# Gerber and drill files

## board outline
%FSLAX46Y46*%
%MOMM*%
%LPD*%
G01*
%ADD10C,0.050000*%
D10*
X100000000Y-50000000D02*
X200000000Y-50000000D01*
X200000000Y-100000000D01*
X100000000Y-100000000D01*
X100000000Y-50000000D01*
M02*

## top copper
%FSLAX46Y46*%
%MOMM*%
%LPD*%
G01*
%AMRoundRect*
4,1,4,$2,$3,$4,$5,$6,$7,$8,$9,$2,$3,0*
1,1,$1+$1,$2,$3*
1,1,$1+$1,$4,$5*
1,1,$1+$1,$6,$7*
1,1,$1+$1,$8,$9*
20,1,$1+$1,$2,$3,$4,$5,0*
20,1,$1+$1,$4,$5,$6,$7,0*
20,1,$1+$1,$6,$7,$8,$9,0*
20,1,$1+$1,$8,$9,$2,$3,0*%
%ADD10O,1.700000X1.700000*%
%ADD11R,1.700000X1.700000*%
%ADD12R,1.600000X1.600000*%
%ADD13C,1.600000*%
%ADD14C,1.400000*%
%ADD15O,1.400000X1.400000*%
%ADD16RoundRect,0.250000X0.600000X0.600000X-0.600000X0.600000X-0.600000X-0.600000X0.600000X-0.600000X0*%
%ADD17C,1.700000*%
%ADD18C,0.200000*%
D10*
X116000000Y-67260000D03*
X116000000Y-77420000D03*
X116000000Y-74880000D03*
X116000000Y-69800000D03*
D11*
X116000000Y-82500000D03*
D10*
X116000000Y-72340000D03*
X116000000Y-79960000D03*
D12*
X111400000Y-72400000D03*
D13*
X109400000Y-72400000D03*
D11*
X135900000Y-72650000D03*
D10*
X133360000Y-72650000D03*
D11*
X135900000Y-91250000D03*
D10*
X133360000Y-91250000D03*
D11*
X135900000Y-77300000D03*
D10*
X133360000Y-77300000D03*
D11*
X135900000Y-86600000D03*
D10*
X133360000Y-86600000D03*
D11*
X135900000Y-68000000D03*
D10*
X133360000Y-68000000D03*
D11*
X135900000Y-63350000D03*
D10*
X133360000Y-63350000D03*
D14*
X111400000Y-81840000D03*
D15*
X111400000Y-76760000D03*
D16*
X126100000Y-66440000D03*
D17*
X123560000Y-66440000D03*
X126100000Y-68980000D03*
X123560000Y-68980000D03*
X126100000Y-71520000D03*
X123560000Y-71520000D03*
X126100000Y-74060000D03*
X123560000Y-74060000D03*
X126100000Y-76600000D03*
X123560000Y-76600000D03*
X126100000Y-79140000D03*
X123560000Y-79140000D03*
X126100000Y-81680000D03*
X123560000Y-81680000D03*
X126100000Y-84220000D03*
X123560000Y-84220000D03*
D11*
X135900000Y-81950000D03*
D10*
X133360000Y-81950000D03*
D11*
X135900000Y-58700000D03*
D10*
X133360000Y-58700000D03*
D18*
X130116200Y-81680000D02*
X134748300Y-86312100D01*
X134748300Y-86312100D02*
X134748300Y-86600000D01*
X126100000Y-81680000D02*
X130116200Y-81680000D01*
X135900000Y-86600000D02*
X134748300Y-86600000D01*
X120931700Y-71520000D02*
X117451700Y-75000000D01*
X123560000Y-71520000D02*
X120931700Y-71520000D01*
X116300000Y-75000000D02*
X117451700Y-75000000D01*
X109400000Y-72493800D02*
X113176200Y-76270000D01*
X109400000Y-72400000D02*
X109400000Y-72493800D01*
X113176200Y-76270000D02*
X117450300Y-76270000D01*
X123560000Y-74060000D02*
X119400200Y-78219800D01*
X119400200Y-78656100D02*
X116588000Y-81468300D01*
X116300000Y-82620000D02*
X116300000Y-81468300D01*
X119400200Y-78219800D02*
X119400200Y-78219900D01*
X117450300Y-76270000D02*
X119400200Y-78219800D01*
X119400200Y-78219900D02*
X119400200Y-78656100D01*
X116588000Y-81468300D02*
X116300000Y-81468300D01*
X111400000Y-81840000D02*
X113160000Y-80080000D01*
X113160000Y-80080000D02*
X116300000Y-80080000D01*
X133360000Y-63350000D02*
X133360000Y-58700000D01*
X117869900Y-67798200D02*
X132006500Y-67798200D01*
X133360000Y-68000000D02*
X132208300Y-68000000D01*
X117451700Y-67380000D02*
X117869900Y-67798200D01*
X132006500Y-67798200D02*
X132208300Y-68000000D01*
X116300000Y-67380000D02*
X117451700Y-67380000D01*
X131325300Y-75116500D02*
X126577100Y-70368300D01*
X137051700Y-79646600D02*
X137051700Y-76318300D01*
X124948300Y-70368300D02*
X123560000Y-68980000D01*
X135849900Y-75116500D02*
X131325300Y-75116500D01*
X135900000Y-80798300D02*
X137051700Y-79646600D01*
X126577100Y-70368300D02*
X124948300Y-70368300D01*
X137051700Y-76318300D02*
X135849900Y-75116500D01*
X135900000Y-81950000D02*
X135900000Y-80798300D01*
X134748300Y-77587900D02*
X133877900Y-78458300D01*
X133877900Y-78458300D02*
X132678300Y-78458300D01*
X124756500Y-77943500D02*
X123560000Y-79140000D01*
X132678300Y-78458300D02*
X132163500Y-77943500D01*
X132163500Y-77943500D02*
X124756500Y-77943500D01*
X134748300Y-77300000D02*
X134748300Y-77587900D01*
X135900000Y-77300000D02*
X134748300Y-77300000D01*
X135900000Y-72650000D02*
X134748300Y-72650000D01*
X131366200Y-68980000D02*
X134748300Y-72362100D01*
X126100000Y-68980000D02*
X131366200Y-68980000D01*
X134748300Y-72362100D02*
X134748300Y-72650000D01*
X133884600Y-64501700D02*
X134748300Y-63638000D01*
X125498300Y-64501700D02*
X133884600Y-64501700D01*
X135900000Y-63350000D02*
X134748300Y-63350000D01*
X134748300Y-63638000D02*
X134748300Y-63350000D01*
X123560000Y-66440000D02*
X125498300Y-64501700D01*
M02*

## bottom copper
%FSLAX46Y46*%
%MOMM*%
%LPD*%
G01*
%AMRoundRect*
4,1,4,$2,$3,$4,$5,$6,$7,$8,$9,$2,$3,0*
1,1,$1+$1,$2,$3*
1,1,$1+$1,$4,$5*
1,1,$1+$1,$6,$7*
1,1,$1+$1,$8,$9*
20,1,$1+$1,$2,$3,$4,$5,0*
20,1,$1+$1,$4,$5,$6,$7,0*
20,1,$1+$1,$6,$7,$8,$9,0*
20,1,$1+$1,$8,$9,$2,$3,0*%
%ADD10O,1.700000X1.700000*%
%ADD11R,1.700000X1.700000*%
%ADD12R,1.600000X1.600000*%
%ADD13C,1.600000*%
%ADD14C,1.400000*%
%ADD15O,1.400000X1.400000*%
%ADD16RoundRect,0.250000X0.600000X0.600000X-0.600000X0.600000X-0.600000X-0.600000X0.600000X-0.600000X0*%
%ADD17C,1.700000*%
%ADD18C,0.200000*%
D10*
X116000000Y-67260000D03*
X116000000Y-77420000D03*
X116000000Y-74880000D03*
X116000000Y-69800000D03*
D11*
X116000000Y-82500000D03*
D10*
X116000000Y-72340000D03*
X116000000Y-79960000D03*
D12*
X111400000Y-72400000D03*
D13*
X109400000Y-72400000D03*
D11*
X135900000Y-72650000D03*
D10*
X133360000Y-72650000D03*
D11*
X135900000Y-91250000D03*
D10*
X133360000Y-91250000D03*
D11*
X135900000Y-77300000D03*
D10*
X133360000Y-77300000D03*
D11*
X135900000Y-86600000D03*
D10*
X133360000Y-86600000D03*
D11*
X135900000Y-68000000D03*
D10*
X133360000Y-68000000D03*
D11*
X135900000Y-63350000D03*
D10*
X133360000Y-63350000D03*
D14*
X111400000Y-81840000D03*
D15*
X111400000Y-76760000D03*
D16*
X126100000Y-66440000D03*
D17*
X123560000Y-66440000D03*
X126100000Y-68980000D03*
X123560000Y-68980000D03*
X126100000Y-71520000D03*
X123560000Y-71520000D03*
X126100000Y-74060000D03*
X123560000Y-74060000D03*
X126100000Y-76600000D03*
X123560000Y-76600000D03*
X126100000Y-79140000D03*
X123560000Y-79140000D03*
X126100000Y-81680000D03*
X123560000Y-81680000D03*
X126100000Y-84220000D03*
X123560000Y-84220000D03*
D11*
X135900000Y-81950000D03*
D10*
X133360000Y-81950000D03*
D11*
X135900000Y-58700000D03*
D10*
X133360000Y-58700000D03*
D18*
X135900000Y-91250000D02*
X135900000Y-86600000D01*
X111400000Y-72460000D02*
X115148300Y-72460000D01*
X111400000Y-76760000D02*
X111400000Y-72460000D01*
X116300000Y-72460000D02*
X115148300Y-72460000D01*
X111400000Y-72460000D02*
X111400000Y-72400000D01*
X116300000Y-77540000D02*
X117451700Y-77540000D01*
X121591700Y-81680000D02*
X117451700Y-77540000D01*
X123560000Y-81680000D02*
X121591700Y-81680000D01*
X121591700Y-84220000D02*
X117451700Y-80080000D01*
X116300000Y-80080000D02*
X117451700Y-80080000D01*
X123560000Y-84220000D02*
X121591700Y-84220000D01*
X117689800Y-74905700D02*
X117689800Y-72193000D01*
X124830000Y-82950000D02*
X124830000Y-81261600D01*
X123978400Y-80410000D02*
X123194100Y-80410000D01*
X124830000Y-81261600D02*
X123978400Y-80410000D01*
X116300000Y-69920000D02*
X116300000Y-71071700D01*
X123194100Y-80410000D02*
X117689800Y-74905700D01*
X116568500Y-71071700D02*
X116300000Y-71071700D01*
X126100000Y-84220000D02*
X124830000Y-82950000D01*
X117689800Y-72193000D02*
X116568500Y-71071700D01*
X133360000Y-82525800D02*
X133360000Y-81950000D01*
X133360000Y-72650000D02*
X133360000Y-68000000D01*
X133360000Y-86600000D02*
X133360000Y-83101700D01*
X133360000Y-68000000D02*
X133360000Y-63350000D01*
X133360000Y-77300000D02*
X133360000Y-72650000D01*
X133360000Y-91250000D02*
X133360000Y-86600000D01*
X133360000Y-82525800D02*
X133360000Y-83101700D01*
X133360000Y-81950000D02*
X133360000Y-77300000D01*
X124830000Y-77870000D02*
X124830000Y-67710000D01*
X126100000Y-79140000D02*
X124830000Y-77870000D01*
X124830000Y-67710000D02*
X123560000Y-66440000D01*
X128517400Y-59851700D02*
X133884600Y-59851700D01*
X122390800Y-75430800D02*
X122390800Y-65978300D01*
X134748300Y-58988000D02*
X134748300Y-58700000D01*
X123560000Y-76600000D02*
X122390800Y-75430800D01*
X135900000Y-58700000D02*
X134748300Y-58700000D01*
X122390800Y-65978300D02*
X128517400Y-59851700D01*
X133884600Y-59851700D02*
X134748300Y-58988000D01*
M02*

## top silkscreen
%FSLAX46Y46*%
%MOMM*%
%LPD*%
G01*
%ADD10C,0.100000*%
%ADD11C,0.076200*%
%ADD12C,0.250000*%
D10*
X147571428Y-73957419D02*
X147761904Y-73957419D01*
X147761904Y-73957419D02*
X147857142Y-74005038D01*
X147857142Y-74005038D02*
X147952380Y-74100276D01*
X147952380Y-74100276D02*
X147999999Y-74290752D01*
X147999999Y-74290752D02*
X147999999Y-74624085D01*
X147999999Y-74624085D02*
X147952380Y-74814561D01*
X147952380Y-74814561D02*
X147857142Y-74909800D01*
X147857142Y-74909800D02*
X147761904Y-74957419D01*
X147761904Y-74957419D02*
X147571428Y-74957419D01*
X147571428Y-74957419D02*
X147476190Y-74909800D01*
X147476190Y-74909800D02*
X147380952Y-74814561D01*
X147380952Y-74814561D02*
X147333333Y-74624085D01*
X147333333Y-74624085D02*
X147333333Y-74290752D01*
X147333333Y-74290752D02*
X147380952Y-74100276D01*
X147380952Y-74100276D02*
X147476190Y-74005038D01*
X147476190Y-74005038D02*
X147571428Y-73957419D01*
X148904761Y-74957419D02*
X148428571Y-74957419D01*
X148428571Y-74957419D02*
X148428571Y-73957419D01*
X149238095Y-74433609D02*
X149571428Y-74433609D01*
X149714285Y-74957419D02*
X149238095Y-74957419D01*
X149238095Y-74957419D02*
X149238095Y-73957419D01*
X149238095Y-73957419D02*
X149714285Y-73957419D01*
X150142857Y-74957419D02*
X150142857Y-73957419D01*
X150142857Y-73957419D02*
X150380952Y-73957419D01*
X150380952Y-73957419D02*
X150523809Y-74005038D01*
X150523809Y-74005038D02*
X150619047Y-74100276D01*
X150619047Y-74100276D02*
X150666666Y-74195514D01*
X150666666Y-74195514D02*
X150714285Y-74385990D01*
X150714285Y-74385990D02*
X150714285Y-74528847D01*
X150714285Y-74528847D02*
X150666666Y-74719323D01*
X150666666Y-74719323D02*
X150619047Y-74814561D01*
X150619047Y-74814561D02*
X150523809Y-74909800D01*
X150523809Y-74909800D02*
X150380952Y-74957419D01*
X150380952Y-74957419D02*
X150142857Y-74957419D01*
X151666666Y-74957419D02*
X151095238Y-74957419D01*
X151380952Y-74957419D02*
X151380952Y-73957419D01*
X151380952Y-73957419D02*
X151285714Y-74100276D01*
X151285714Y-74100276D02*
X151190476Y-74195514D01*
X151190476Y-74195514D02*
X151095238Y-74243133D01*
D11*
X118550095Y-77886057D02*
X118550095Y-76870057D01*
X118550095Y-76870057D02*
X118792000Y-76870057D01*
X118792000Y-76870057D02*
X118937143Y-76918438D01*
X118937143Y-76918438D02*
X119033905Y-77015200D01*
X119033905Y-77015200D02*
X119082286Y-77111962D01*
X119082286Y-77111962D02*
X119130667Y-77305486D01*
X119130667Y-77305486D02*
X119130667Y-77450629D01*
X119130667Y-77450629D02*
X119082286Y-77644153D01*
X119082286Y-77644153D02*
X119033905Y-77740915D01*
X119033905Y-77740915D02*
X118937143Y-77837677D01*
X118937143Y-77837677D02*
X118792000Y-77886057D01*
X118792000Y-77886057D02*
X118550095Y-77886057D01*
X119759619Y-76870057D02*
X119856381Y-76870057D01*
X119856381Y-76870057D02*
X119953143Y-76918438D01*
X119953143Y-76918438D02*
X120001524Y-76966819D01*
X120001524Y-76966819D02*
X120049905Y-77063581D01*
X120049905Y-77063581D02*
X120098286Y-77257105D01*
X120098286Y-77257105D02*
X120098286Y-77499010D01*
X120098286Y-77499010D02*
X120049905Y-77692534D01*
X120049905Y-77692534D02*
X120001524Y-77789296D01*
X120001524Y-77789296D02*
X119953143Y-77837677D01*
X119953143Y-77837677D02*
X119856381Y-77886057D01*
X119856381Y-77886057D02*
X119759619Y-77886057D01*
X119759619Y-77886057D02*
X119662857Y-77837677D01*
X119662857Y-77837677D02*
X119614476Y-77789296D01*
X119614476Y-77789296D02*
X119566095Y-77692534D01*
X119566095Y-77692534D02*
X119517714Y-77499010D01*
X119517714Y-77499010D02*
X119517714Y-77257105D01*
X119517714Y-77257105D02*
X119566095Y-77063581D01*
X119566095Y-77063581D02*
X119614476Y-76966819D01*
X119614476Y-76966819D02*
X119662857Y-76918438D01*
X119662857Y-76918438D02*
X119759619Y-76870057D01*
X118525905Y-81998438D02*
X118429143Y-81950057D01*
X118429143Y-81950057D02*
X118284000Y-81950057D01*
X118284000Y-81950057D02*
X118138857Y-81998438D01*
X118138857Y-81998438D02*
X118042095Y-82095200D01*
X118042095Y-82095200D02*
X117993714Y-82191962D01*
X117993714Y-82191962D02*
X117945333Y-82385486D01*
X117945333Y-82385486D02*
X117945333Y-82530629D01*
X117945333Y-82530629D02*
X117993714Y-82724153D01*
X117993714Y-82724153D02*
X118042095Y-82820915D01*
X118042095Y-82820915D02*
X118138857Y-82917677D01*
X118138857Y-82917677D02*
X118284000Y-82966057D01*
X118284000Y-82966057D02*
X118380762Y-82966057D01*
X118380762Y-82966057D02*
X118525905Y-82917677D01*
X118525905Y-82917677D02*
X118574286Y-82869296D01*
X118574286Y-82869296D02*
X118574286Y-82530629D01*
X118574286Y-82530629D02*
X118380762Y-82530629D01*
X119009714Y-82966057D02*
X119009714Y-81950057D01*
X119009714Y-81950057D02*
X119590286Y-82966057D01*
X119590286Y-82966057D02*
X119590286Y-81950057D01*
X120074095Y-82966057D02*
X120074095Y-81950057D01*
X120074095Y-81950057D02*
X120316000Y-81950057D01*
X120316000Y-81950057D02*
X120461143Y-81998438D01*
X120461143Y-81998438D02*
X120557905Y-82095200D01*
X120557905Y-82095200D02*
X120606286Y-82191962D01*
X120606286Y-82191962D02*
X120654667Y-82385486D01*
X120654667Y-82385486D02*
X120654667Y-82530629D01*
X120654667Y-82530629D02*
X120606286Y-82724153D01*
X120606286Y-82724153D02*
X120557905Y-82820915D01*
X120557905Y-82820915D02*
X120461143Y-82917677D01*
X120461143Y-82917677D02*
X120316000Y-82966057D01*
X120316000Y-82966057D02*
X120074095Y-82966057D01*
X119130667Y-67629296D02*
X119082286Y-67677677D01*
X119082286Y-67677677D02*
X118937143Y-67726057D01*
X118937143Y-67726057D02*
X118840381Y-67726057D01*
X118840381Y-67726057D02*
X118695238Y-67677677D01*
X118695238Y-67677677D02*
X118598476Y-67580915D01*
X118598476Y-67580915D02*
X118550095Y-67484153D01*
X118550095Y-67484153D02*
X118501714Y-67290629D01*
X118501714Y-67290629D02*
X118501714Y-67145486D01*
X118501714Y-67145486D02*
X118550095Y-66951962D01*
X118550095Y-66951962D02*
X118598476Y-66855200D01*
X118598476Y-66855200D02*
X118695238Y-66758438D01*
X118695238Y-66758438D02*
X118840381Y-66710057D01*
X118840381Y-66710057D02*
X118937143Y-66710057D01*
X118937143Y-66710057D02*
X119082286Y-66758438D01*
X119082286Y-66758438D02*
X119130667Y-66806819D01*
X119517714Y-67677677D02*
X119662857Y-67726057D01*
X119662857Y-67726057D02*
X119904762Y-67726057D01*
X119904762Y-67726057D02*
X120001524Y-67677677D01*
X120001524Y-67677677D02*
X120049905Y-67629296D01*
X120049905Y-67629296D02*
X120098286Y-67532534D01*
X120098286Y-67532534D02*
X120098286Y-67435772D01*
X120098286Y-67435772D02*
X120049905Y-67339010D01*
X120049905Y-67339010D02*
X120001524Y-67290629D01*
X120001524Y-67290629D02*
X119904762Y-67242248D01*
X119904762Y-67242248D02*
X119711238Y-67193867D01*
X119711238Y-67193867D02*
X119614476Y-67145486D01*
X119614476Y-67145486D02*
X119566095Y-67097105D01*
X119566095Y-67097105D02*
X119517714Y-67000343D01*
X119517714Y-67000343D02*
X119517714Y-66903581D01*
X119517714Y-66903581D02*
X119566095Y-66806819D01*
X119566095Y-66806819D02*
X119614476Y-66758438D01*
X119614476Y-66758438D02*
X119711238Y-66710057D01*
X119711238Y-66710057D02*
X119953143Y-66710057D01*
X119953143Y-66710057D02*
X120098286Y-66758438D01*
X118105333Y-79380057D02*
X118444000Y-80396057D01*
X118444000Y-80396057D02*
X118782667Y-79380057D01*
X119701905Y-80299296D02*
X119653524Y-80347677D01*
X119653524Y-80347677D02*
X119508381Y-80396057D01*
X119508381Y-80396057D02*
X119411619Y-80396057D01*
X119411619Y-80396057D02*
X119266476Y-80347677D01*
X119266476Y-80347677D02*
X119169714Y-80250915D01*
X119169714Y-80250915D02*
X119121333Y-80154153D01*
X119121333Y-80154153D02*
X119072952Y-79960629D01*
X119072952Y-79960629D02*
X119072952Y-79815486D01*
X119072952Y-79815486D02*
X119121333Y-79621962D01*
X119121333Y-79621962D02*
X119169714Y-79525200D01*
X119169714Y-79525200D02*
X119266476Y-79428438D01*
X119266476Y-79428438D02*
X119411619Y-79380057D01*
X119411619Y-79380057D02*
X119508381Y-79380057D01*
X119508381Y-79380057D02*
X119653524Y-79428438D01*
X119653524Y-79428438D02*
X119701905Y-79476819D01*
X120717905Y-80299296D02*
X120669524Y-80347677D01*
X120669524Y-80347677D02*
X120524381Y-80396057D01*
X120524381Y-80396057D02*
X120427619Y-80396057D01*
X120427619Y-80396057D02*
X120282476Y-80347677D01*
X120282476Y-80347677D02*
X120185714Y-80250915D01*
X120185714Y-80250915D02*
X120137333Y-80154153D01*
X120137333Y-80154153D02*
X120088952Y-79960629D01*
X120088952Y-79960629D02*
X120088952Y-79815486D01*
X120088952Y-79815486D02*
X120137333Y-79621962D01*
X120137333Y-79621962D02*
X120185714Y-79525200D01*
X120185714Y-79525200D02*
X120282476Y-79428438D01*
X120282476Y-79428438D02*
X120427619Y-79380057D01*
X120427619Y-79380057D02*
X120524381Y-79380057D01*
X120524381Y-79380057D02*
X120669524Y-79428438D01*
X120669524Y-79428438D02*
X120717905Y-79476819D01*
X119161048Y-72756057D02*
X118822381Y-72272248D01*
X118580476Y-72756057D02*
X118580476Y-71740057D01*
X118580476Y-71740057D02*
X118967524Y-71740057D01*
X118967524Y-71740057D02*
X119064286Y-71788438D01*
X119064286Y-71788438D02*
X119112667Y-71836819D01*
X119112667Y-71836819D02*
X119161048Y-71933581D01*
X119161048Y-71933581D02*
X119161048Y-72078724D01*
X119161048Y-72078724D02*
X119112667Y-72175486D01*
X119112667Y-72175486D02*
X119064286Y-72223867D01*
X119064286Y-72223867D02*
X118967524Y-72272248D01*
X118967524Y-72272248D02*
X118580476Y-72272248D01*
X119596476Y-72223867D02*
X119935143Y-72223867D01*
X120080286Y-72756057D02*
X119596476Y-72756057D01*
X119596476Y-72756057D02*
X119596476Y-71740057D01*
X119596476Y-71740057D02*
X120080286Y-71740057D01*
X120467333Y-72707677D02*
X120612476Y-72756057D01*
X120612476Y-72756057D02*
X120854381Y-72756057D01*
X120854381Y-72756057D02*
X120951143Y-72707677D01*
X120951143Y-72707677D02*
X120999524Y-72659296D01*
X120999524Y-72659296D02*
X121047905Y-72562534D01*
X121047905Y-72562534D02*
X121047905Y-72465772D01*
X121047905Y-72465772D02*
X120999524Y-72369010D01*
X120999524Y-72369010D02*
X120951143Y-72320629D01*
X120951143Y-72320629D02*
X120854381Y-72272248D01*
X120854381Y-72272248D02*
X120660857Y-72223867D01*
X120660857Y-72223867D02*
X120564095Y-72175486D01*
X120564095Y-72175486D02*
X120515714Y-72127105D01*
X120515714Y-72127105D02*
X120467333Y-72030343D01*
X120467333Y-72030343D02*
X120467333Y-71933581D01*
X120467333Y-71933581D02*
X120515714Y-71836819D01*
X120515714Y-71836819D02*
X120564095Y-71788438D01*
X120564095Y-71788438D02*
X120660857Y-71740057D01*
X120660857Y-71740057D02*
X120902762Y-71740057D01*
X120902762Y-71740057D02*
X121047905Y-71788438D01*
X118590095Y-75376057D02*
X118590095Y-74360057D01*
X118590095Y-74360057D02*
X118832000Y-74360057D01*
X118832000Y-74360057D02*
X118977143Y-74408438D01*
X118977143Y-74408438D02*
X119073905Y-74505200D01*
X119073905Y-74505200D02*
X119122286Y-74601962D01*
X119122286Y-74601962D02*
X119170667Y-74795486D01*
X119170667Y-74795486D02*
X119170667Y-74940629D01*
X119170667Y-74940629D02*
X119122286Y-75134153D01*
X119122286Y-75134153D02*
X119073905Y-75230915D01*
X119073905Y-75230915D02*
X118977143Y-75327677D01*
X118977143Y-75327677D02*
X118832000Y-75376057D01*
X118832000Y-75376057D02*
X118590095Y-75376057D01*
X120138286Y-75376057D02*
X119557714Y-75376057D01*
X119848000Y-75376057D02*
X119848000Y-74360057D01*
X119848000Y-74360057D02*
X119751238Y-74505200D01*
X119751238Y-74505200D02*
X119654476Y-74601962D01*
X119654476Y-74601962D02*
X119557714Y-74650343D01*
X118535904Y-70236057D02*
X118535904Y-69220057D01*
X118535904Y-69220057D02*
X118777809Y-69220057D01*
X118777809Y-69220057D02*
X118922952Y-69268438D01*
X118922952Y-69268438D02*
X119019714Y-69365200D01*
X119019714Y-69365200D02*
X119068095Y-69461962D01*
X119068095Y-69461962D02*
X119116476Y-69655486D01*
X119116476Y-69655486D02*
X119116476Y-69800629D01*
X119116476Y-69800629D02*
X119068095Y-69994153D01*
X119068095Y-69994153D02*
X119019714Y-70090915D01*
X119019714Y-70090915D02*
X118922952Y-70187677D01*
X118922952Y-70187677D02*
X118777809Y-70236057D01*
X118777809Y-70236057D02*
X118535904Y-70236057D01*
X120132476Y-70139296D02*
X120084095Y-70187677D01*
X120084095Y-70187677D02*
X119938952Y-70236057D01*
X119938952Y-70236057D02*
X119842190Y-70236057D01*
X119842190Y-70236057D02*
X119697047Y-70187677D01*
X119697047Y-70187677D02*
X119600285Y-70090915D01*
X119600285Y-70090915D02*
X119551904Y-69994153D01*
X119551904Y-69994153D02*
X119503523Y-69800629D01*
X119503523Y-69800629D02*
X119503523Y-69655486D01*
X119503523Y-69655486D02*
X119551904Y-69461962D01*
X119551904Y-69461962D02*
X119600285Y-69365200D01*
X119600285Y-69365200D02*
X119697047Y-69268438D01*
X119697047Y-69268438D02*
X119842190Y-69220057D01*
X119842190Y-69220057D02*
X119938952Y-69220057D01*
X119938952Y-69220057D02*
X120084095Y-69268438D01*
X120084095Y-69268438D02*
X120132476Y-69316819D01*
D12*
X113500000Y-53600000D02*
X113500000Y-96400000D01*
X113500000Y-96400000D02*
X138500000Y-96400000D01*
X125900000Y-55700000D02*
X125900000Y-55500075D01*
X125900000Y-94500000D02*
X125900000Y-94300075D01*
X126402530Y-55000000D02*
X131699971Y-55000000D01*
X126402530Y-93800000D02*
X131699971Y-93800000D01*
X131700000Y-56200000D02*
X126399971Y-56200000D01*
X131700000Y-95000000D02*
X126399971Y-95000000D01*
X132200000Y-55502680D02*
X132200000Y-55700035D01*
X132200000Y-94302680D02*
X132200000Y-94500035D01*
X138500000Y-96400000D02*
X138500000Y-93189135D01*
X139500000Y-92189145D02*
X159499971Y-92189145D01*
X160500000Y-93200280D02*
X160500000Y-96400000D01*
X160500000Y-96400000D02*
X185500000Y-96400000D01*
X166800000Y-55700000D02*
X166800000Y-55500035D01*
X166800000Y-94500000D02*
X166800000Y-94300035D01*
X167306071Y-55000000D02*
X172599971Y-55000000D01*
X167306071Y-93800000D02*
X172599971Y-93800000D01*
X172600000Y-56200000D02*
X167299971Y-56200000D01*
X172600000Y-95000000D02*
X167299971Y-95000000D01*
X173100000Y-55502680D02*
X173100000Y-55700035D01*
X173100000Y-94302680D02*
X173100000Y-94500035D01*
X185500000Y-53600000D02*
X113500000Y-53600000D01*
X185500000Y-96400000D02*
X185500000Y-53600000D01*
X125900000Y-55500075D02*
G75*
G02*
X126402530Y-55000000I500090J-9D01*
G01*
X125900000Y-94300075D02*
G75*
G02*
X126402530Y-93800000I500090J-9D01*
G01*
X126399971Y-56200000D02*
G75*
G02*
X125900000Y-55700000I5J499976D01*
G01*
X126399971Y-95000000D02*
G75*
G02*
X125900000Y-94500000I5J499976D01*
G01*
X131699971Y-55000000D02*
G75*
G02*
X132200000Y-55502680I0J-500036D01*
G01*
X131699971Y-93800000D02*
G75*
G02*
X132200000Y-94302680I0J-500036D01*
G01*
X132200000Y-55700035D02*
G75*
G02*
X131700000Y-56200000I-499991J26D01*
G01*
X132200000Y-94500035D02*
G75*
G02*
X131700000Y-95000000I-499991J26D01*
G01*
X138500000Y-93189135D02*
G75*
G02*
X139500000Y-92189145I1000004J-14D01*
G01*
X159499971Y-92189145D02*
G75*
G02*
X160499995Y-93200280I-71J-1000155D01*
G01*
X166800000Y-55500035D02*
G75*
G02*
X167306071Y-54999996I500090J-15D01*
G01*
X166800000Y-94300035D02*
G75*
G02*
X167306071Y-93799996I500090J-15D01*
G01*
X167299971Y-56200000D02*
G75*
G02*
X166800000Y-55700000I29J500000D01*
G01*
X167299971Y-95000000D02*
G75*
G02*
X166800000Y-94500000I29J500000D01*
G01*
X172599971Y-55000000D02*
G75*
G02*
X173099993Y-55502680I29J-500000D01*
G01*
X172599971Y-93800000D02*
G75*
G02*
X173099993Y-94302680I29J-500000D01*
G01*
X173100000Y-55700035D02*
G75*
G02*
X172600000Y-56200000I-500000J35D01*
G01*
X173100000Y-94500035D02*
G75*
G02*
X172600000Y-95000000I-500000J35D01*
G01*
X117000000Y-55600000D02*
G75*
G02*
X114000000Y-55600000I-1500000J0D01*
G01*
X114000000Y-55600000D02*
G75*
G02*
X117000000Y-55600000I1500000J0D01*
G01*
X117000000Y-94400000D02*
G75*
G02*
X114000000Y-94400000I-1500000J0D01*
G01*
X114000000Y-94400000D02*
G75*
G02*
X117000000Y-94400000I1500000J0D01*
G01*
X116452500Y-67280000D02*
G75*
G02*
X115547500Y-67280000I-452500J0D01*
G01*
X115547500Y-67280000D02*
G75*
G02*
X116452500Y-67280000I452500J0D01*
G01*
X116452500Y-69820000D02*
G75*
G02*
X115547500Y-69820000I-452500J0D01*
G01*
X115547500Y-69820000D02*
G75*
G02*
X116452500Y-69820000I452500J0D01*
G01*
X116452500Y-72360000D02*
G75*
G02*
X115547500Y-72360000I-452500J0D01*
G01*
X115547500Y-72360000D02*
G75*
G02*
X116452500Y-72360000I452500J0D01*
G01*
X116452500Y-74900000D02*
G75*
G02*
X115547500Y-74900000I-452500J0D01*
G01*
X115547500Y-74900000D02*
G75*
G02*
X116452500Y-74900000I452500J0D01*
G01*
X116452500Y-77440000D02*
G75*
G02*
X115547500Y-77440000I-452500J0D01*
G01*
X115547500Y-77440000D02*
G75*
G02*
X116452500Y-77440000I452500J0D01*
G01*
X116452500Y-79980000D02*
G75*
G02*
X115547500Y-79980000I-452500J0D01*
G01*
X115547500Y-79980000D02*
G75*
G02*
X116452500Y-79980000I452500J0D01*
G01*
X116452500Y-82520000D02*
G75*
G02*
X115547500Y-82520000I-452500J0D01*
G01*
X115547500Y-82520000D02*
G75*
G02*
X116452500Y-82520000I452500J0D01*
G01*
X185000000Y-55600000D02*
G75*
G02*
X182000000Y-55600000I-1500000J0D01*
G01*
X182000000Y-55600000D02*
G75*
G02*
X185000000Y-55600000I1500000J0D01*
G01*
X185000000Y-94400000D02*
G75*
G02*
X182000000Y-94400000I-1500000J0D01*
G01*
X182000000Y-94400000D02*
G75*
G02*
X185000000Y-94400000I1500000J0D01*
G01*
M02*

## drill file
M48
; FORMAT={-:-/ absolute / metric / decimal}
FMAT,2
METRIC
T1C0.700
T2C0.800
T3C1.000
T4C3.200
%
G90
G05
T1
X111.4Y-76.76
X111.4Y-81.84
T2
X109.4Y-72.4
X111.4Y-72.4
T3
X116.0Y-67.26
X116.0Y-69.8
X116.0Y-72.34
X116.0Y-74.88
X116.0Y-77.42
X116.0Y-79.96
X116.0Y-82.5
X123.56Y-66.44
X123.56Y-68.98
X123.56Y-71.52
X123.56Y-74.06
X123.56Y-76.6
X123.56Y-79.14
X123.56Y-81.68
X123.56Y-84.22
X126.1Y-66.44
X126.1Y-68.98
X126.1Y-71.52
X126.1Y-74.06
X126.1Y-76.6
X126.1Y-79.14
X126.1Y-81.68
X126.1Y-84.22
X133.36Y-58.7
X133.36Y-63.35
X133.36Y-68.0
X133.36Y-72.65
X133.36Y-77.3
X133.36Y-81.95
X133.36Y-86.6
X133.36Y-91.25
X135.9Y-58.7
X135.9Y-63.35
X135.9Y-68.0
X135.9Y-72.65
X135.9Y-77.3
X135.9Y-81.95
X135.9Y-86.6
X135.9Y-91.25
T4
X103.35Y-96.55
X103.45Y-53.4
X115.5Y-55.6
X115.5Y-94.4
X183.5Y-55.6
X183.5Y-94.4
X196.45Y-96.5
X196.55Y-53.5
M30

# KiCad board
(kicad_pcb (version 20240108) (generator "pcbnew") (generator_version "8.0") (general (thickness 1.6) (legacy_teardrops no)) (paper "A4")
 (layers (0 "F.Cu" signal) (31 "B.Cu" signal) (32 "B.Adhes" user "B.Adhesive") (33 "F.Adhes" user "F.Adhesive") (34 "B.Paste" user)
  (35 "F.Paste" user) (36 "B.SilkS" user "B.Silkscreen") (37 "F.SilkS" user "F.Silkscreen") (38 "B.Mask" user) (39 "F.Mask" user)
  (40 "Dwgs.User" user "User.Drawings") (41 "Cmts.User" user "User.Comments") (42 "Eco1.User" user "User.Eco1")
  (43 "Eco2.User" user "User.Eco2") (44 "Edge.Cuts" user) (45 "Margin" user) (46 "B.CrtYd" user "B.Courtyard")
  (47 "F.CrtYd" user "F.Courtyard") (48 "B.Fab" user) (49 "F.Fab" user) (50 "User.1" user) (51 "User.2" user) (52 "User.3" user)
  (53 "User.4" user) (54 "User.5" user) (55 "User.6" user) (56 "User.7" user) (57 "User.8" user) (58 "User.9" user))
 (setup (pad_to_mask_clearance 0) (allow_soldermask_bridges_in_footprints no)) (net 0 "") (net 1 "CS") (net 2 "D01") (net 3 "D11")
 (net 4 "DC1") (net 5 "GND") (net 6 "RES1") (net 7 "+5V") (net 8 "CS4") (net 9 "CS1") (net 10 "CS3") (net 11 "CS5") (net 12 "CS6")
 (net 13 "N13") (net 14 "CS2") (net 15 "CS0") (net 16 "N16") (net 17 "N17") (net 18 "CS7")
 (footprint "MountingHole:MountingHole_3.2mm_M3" (layer "F.Cu") (at 183.5 55.6)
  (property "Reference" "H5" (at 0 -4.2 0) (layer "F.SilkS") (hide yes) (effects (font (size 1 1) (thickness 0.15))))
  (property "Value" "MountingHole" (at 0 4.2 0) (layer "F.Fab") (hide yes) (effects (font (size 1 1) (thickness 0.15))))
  (pad "" np_thru_hole circle (at 0 0) (size 3.2 3.2) (drill 3.2) (layers "*.Cu" "*.Mask")))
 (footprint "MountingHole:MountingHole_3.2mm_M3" (layer "F.Cu") (at 183.5 94.4)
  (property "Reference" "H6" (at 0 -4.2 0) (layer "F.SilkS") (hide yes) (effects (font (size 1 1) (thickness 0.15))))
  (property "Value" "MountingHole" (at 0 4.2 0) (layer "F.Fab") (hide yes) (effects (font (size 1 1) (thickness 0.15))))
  (pad "" np_thru_hole circle (at 0 0) (size 3.2 3.2) (drill 3.2) (layers "*.Cu" "*.Mask")))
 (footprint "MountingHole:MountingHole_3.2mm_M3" (layer "F.Cu") (at 196.55 53.5)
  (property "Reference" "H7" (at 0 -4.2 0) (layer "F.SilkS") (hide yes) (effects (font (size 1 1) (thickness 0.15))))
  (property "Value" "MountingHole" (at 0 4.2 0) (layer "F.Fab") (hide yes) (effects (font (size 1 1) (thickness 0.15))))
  (pad "" np_thru_hole circle (at 0 0) (size 3.2 3.2) (drill 3.2) (layers "*.Cu" "*.Mask")))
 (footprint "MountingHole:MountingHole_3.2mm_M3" (layer "F.Cu") (at 115.5 55.6)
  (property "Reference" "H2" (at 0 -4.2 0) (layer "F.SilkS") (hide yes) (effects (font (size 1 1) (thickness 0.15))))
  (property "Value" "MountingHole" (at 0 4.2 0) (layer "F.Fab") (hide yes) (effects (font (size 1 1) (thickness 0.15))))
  (pad "" np_thru_hole circle (at 0 0) (size 3.2 3.2) (drill 3.2) (layers "*.Cu" "*.Mask")))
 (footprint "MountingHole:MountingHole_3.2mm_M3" (layer "F.Cu") (at 103.35 96.55)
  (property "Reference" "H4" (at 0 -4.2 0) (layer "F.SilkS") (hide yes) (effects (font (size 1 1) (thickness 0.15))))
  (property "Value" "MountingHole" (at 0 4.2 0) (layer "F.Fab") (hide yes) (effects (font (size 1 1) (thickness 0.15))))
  (pad "" np_thru_hole circle (at 0 0) (size 3.2 3.2) (drill 3.2) (layers "*.Cu" "*.Mask")))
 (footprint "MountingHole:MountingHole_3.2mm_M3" (layer "F.Cu") (at 103.45 53.4)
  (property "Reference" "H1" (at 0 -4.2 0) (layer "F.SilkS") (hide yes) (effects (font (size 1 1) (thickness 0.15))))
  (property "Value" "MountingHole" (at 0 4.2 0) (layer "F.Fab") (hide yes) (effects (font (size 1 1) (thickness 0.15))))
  (pad "" np_thru_hole circle (at 0 0) (size 3.2 3.2) (drill 3.2) (layers "*.Cu" "*.Mask")))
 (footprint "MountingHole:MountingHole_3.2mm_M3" (layer "F.Cu") (at 115.5 94.4)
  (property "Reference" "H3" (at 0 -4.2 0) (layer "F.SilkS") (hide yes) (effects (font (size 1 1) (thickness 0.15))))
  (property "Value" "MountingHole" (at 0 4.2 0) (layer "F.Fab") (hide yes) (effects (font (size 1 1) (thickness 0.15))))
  (pad "" np_thru_hole circle (at 0 0) (size 3.2 3.2) (drill 3.2) (layers "*.Cu" "*.Mask")))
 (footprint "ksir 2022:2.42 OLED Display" (layer "F.Cu") (at 149.5 75)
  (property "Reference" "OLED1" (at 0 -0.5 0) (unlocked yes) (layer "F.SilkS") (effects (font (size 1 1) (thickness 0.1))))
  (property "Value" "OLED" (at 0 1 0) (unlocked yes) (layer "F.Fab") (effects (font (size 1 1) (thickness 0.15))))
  (fp_line (start -36 -21.4) (end -36 21.4) (stroke (width 0.25) (type default)) (layer "F.SilkS"))
  (fp_line (start -36 21.4) (end -11 21.4) (stroke (width 0.25) (type default)) (layer "F.SilkS"))
  (fp_line (start -23.6 -19.3) (end -23.6 -19.499925) (stroke (width 0.25) (type default)) (layer "F.SilkS"))
  (fp_line (start -23.6 19.5) (end -23.6 19.300075) (stroke (width 0.25) (type default)) (layer "F.SilkS"))
  (fp_line (start -23.09747 -20) (end -17.800029 -20) (stroke (width 0.25) (type default)) (layer "F.SilkS"))
  (fp_line (start -23.09747 18.8) (end -17.800029 18.8) (stroke (width 0.25) (type default)) (layer "F.SilkS"))
  (fp_line (start -17.8 -18.8) (end -23.100029 -18.8) (stroke (width 0.25) (type default)) (layer "F.SilkS"))
  (fp_line (start -17.8 20) (end -23.100029 20) (stroke (width 0.25) (type default)) (layer "F.SilkS"))
  (fp_line (start -17.3 -19.49732) (end -17.3 -19.299965) (stroke (width 0.25) (type default)) (layer "F.SilkS"))
  (fp_line (start -17.3 19.30268) (end -17.3 19.500035) (stroke (width 0.25) (type default)) (layer "F.SilkS"))
  (fp_line (start -11 21.4) (end -11 18.189135) (stroke (width 0.25) (type default)) (layer "F.SilkS"))
  (fp_line (start -10 17.189145) (end 9.999971 17.189145) (stroke (width 0.25) (type default)) (layer "F.SilkS"))
  (fp_line (start 11 18.20028) (end 11 21.4) (stroke (width 0.25) (type default)) (layer "F.SilkS"))
  (fp_line (start 11 21.4) (end 36 21.4) (stroke (width 0.25) (type default)) (layer "F.SilkS"))
  (fp_line (start 17.3 -19.3) (end 17.3 -19.499965) (stroke (width 0.25) (type default)) (layer "F.SilkS"))
  (fp_line (start 17.3 19.5) (end 17.3 19.300035) (stroke (width 0.25) (type default)) (layer "F.SilkS"))
  (fp_line (start 17.806071 -20) (end 23.099971 -20) (stroke (width 0.25) (type default)) (layer "F.SilkS"))
  (fp_line (start 17.806071 18.8) (end 23.099971 18.8) (stroke (width 0.25) (type default)) (layer "F.SilkS"))
  (fp_line (start 23.1 -18.8) (end 17.799971 -18.8) (stroke (width 0.25) (type default)) (layer "F.SilkS"))
  (fp_line (start 23.1 20) (end 17.799971 20) (stroke (width 0.25) (type default)) (layer "F.SilkS"))
  (fp_line (start 23.6 -19.49732) (end 23.6 -19.299965) (stroke (width 0.25) (type default)) (layer "F.SilkS"))
  (fp_line (start 23.6 19.30268) (end 23.6 19.500035) (stroke (width 0.25) (type default)) (layer "F.SilkS"))
  (fp_line (start 36 -21.4) (end -36 -21.4) (stroke (width 0.25) (type default)) (layer "F.SilkS"))
  (fp_line (start 36 21.4) (end 36 -21.4) (stroke (width 0.25) (type default)) (layer "F.SilkS"))
  (fp_arc (start -23.6 -19.499925) (mid -23.45266 -19.854398) (end -23.09747 -20) (stroke (width 0.25) (type default)) (layer "F.SilkS"))
  (fp_arc (start -23.6 19.300075) (mid -23.45266 18.945602) (end -23.09747 18.8) (stroke (width 0.25) (type default)) (layer "F.SilkS"))
  (fp_arc (start -23.100029 -18.8) (mid -23.453571 -18.94645) (end -23.6 -19.3) (stroke (width 0.25) (type default)) (layer "F.SilkS"))
  (fp_arc (start -23.100029 20) (mid -23.453571 19.85355) (end -23.6 19.5) (stroke (width 0.25) (type default)) (layer "F.SilkS"))
  (fp_arc (start -17.800029 -20) (mid -17.445517 -19.852607) (end -17.3 -19.49732) (stroke (width 0.25) (type default)) (layer "F.SilkS"))
  (fp_arc (start -17.800029 18.8) (mid -17.445517 18.947393) (end -17.3 19.30268) (stroke (width 0.25) (type default)) (layer "F.SilkS"))
  (fp_arc (start -17.3 -19.299965) (mid -17.446456 -18.946432) (end -17.8 -18.8) (stroke (width 0.25) (type default)) (layer "F.SilkS"))
  (fp_arc (start -17.3 19.500035) (mid -17.446456 19.853568) (end -17.8 20) (stroke (width 0.25) (type default)) (layer "F.SilkS"))
  (fp_arc (start -11 18.189135) (mid -10.707102 17.482036) (end -10 17.189145) (stroke (width 0.25) (type default)) (layer "F.SilkS"))
  (fp_arc (start 9.999971 17.189145) (mid 10.711013 17.486002) (end 11 18.20028) (stroke (width 0.25) (type default)) (layer "F.SilkS"))
  (fp_arc (start 17.3 -19.499965) (mid 17.44861 -19.855688) (end 17.806071 -20) (stroke (width 0.25) (type default)) (layer "F.SilkS"))
  (fp_arc (start 17.3 19.300035) (mid 17.44861 18.944312) (end 17.806071 18.8) (stroke (width 0.25) (type default)) (layer "F.SilkS"))
  (fp_arc (start 17.799971 -18.8) (mid 17.446436 -18.946457) (end 17.3 -19.3) (stroke (width 0.25) (type default)) (layer "F.SilkS"))
  (fp_arc (start 17.799971 20) (mid 17.446436 19.853543) (end 17.3 19.5) (stroke (width 0.25) (type default)) (layer "F.SilkS"))
  (fp_arc (start 23.099971 -20) (mid 23.454489 -19.852615) (end 23.6 -19.49732) (stroke (width 0.25) (type default)) (layer "F.SilkS"))
  (fp_arc (start 23.099971 18.8) (mid 23.454489 18.947385) (end 23.6 19.30268) (stroke (width 0.25) (type default)) (layer "F.SilkS"))
  (fp_arc (start 23.6 -19.299965) (mid 23.453541 -18.946434) (end 23.1 -18.8) (stroke (width 0.25) (type default)) (layer "F.SilkS"))
  (fp_arc (start 23.6 19.500035) (mid 23.453541 19.853566) (end 23.1 20) (stroke (width 0.25) (type default)) (layer "F.SilkS"))
  (fp_circle (center -34 -19.4) (end -32.5 -19.4) (stroke (width 0.25) (type default)) (fill none) (layer "F.SilkS"))
  (fp_circle (center -34 19.4) (end -32.5 19.4) (stroke (width 0.25) (type default)) (fill none) (layer "F.SilkS"))
  (fp_circle (center -33.5 -7.72) (end -33.0475 -7.72) (stroke (width 0.25) (type default)) (fill none) (layer "F.SilkS"))
  (fp_circle (center -33.5 -5.18) (end -33.0475 -5.18) (stroke (width 0.25) (type default)) (fill none) (layer "F.SilkS"))
  (fp_circle (center -33.5 -2.64) (end -33.0475 -2.64) (stroke (width 0.25) (type default)) (fill none) (layer "F.SilkS"))
  (fp_circle (center -33.5 -0.1) (end -33.0475 -0.1) (stroke (width 0.25) (type default)) (fill none) (layer "F.SilkS"))
  (fp_circle (center -33.5 2.44) (end -33.0475 2.44) (stroke (width 0.25) (type default)) (fill none) (layer "F.SilkS"))
  (fp_circle (center -33.5 4.98) (end -33.0475 4.98) (stroke (width 0.25) (type default)) (fill none) (layer "F.SilkS"))
  (fp_circle (center -33.5 7.52) (end -33.0475 7.52) (stroke (width 0.25) (type default)) (fill none) (layer "F.SilkS"))
  (fp_circle (center 34 -19.4) (end 35.5 -19.4) (stroke (width 0.25) (type default)) (fill none) (layer "F.SilkS"))
  (fp_circle (center 34 19.4) (end 35.5 19.4) (stroke (width 0.25) (type default)) (fill none) (layer "F.SilkS"))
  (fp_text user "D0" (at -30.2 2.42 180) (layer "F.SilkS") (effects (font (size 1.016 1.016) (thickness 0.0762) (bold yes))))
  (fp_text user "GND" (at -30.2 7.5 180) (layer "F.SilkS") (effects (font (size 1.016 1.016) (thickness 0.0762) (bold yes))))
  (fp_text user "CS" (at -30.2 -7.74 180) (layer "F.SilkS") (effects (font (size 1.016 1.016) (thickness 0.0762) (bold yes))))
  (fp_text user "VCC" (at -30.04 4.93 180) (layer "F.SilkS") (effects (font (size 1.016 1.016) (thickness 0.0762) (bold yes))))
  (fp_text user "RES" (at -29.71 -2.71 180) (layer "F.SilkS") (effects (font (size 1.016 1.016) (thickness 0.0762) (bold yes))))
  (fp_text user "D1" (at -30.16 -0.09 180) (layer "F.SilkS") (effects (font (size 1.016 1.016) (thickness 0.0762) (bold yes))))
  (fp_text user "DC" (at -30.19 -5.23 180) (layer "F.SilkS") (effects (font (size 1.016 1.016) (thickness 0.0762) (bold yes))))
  (pad "CS" thru_hole oval (at -33.5 -7.74 180) (size 1.7 1.7) (drill 1) (layers "*.Cu" "*.Mask") (remove_unused_layers no) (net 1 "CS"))
  (pad "D0" thru_hole oval (at -33.5 2.42 180) (size 1.7 1.7) (drill 1) (layers "*.Cu" "*.Mask") (remove_unused_layers no) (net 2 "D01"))
  (pad "D1" thru_hole oval (at -33.5 -0.12 180) (size 1.7 1.7) (drill 1) (layers "*.Cu" "*.Mask") (remove_unused_layers no) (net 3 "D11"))
  (pad "DC" thru_hole oval (at -33.5 -5.2 180) (size 1.7 1.7) (drill 1) (layers "*.Cu" "*.Mask") (remove_unused_layers no) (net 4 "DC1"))
  (pad "GND" thru_hole rect (at -33.5 7.5 180) (size 1.7 1.7) (drill 1) (layers "*.Cu" "*.Mask") (remove_unused_layers no) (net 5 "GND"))
  (pad "RES" thru_hole oval (at -33.5 -2.66 180) (size 1.7 1.7) (drill 1) (layers "*.Cu" "*.Mask") (remove_unused_layers no) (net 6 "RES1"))
  (pad "VCC" thru_hole oval (at -33.5 4.96 180) (size 1.7 1.7) (drill 1) (layers "*.Cu" "*.Mask") (remove_unused_layers no) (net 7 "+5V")))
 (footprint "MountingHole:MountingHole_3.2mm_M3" (layer "F.Cu") (at 196.45 96.5)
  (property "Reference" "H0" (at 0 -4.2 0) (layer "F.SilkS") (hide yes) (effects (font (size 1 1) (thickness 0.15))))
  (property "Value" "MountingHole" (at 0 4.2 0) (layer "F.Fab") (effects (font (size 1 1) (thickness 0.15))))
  (pad "" np_thru_hole circle (at 0 0) (size 3.2 3.2) (drill 3.2) (layers "*.Cu" "*.Mask")))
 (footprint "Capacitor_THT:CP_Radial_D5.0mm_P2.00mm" (layer "B.Cu") (at 111.4 72.4 180)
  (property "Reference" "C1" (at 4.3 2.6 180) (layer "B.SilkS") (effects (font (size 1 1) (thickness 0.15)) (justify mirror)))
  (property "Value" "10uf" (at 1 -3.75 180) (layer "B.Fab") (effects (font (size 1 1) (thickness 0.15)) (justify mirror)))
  (pad "1" thru_hole rect (at 0 0 180) (size 1.6 1.6) (drill 0.8) (layers "*.Cu" "*.Mask") (remove_unused_layers no) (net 6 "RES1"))
  (pad "2" thru_hole circle (at 2 0 180) (size 1.6 1.6) (drill 0.8) (layers "*.Cu" "*.Mask") (remove_unused_layers no) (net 5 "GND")))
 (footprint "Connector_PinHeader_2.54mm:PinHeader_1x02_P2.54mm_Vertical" (layer "B.Cu") (at 135.9 72.65 90)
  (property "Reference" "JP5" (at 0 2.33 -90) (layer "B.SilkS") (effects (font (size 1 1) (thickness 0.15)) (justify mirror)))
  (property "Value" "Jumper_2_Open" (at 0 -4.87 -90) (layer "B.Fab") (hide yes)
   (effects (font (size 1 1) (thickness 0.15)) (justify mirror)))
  (pad "1" thru_hole rect (at 0 0 90) (size 1.7 1.7) (drill 1) (layers "*.Cu" "*.Mask") (remove_unused_layers no) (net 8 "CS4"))
  (pad "2" thru_hole oval (at 0 -2.54 90) (size 1.7 1.7) (drill 1) (layers "*.Cu" "*.Mask") (remove_unused_layers no) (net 1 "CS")))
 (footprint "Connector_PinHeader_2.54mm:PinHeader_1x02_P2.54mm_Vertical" (layer "B.Cu") (at 135.9 91.25 90)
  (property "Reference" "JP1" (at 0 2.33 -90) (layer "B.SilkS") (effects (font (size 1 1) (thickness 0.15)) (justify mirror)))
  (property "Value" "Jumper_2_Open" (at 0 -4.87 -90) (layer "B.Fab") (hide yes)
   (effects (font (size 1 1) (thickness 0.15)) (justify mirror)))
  (pad "1" thru_hole rect (at 0 0 90) (size 1.7 1.7) (drill 1) (layers "*.Cu" "*.Mask") (remove_unused_layers no) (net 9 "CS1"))
  (pad "2" thru_hole oval (at 0 -2.54 90) (size 1.7 1.7) (drill 1) (layers "*.Cu" "*.Mask") (remove_unused_layers no) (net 1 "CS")))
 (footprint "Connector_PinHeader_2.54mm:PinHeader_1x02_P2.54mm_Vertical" (layer "B.Cu") (at 135.9 77.3 90)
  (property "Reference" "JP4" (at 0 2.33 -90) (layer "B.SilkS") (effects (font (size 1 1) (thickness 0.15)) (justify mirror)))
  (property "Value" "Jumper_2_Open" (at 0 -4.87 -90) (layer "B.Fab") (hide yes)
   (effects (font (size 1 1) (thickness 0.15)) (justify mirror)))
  (pad "1" thru_hole rect (at 0 0 90) (size 1.7 1.7) (drill 1) (layers "*.Cu" "*.Mask") (remove_unused_layers no) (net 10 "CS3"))
  (pad "2" thru_hole oval (at 0 -2.54 90) (size 1.7 1.7) (drill 1) (layers "*.Cu" "*.Mask") (remove_unused_layers no) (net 1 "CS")))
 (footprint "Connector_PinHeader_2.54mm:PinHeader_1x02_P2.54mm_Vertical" (layer "B.Cu") (at 135.9 86.6 90)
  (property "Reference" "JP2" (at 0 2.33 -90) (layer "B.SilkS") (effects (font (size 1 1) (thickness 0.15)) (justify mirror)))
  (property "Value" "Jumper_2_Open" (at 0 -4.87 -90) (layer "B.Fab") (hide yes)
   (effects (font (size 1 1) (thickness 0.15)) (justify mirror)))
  (pad "1" thru_hole rect (at 0 0 90) (size 1.7 1.7) (drill 1) (layers "*.Cu" "*.Mask") (remove_unused_layers no) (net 9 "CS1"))
  (pad "2" thru_hole oval (at 0 -2.54 90) (size 1.7 1.7) (drill 1) (layers "*.Cu" "*.Mask") (remove_unused_layers no) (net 1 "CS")))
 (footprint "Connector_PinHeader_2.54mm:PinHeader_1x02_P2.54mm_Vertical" (layer "B.Cu") (at 135.9 68 90)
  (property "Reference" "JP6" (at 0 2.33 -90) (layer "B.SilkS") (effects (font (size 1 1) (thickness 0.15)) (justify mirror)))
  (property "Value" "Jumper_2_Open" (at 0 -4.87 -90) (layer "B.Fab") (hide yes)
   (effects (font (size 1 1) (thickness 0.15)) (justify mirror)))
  (pad "1" thru_hole rect (at 0 0 90) (size 1.7 1.7) (drill 1) (layers "*.Cu" "*.Mask") (remove_unused_layers no) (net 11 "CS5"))
  (pad "2" thru_hole oval (at 0 -2.54 90) (size 1.7 1.7) (drill 1) (layers "*.Cu" "*.Mask") (remove_unused_layers no) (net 1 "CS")))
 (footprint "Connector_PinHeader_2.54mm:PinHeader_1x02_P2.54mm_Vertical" (layer "B.Cu") (at 135.9 63.35 90)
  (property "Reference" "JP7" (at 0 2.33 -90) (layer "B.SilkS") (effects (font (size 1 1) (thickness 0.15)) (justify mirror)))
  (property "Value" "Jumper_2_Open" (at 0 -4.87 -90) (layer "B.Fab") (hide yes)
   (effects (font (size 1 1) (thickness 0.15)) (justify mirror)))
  (pad "1" thru_hole rect (at 0 0 90) (size 1.7 1.7) (drill 1) (layers "*.Cu" "*.Mask") (remove_unused_layers no) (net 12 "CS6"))
  (pad "2" thru_hole oval (at 0 -2.54 90) (size 1.7 1.7) (drill 1) (layers "*.Cu" "*.Mask") (remove_unused_layers no) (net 1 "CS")))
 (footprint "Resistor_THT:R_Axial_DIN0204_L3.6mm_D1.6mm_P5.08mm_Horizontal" (layer "B.Cu") (at 111.4 81.84 90)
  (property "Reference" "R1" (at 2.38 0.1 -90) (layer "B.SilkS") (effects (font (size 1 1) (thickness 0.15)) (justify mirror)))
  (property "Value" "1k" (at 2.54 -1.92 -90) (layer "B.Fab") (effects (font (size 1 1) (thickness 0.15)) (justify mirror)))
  (pad "1" thru_hole circle (at 0 0 90) (size 1.4 1.4) (drill 0.7) (layers "*.Cu" "*.Mask") (remove_unused_layers no) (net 7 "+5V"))
  (pad "2" thru_hole oval (at 5.08 0 90) (size 1.4 1.4) (drill 0.7) (layers "*.Cu" "*.Mask") (remove_unused_layers no) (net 6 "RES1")))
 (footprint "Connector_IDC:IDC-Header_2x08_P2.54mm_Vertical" (layer "B.Cu") (at 126.1 66.44 180)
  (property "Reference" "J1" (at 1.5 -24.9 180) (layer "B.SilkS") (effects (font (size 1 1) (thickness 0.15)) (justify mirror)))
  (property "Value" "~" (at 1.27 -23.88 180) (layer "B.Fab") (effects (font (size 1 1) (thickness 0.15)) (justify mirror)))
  (pad "1" thru_hole roundrect (at 0 0 180) (size 1.7 1.7) (drill 1) (layers "*.Cu" "*.Mask") (remove_unused_layers no)
   (roundrect_rratio 0.147059) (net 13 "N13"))
  (pad "2" thru_hole circle (at 2.54 0 180) (size 1.7 1.7) (drill 1) (layers "*.Cu" "*.Mask") (remove_unused_layers no) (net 12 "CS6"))
  (pad "3" thru_hole circle (at 0 -2.54 180) (size 1.7 1.7) (drill 1) (layers "*.Cu" "*.Mask") (remove_unused_layers no) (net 8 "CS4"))
  (pad "4" thru_hole circle (at 2.54 -2.54 180) (size 1.7 1.7) (drill 1) (layers "*.Cu" "*.Mask") (remove_unused_layers no) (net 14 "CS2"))
  (pad "5" thru_hole circle (at 0 -5.08 180) (size 1.7 1.7) (drill 1) (layers "*.Cu" "*.Mask") (remove_unused_layers no) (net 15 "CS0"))
  (pad "6" thru_hole circle (at 2.54 -5.08 180) (size 1.7 1.7) (drill 1) (layers "*.Cu" "*.Mask") (remove_unused_layers no) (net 3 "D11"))
  (pad "7" thru_hole circle (at 0 -7.62 180) (size 1.7 1.7) (drill 1) (layers "*.Cu" "*.Mask") (remove_unused_layers no) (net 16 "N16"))
  (pad "8" thru_hole circle (at 2.54 -7.62 180) (size 1.7 1.7) (drill 1) (layers "*.Cu" "*.Mask") (remove_unused_layers no) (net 5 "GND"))
  (pad "9" thru_hole circle (at 0 -10.16 180) (size 1.7 1.7) (drill 1) (layers "*.Cu" "*.Mask") (remove_unused_layers no) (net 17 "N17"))
  (pad "10" thru_hole circle (at 2.54 -10.16 180) (size 1.7 1.7) (drill 1) (layers "*.Cu" "*.Mask") (remove_unused_layers no) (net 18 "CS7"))
  (pad "11" thru_hole circle (at 0 -12.7 180) (size 1.7 1.7) (drill 1) (layers "*.Cu" "*.Mask") (remove_unused_layers no) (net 12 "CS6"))
  (pad "12" thru_hole circle (at 2.54 -12.7 180) (size 1.7 1.7) (drill 1) (layers "*.Cu" "*.Mask") (remove_unused_layers no) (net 10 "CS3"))
  (pad "13" thru_hole circle (at 0 -15.24 180) (size 1.7 1.7) (drill 1) (layers "*.Cu" "*.Mask") (remove_unused_layers no) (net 9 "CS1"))
  (pad "14" thru_hole circle (at 2.54 -15.24 180) (size 1.7 1.7) (drill 1) (layers "*.Cu" "*.Mask") (remove_unused_layers no) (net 2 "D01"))
  (pad "15" thru_hole circle (at 0 -17.78 180) (size 1.7 1.7) (drill 1) (layers "*.Cu" "*.Mask") (remove_unused_layers no) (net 4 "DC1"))
  (pad "16" thru_hole circle (at 2.54 -17.78 180) (size 1.7 1.7) (drill 1) (layers "*.Cu" "*.Mask") (remove_unused_layers no) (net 7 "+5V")))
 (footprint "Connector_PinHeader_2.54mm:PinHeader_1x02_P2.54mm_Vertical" (layer "B.Cu") (at 135.9 81.95 90)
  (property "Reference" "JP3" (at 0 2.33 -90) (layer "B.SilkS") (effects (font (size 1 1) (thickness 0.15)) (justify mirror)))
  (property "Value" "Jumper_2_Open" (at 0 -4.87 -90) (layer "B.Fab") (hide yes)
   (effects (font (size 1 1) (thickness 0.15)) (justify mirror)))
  (pad "1" thru_hole rect (at 0 0 90) (size 1.7 1.7) (drill 1) (layers "*.Cu" "*.Mask") (remove_unused_layers no) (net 14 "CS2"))
  (pad "2" thru_hole oval (at 0 -2.54 90) (size 1.7 1.7) (drill 1) (layers "*.Cu" "*.Mask") (remove_unused_layers no) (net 1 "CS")))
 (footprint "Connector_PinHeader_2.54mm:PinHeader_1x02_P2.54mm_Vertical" (layer "B.Cu") (at 135.9 58.7 90)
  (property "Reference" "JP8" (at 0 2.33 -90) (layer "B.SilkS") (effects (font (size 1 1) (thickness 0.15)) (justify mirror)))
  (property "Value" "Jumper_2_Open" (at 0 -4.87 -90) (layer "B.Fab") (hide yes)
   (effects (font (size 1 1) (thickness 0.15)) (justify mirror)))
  (pad "1" thru_hole rect (at 0 0 90) (size 1.7 1.7) (drill 1) (layers "*.Cu" "*.Mask") (remove_unused_layers no) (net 18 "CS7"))
  (pad "2" thru_hole oval (at 0 -2.54 90) (size 1.7 1.7) (drill 1) (layers "*.Cu" "*.Mask") (remove_unused_layers no) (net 1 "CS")))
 (gr_rect (start 100 50) (end 200 100) (stroke (width 0.05) (type default)) (fill none) (layer "Edge.Cuts"))
 (segment (start 130.1162 81.68) (end 134.7483 86.3121) (width 0.2) (layer "F.Cu") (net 9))
 (segment (start 134.7483 86.3121) (end 134.7483 86.6) (width 0.2) (layer "F.Cu") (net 9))
 (segment (start 126.1 81.68) (end 130.1162 81.68) (width 0.2) (layer "F.Cu") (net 9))
 (segment (start 135.9 86.6) (end 134.7483 86.6) (width 0.2) (layer "F.Cu") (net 9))
 (segment (start 135.9 91.25) (end 135.9 86.6) (width 0.2) (layer "B.Cu") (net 9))
 (segment (start 120.9317 71.52) (end 117.4517 75) (width 0.2) (layer "F.Cu") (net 3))
 (segment (start 123.56 71.52) (end 120.9317 71.52) (width 0.2) (layer "F.Cu") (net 3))
 (segment (start 116.3 75) (end 117.4517 75) (width 0.2) (layer "F.Cu") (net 3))
 (segment (start 109.4 72.4938) (end 113.1762 76.27) (width 0.2) (layer "F.Cu") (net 5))
 (segment (start 109.4 72.4) (end 109.4 72.4938) (width 0.2) (layer "F.Cu") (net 5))
 (segment (start 113.1762 76.27) (end 117.4503 76.27) (width 0.2) (layer "F.Cu") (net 5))
 (segment (start 123.56 74.06) (end 119.4002 78.2198) (width 0.2) (layer "F.Cu") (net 5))
 (segment (start 119.4002 78.6561) (end 116.588 81.4683) (width 0.2) (layer "F.Cu") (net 5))
 (segment (start 116.3 82.62) (end 116.3 81.4683) (width 0.2) (layer "F.Cu") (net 5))
 (segment (start 119.4002 78.2198) (end 119.4002 78.2199) (width 0.2) (layer "F.Cu") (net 5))
 (segment (start 117.4503 76.27) (end 119.4002 78.2198) (width 0.2) (layer "F.Cu") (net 5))
 (segment (start 119.4002 78.2199) (end 119.4002 78.6561) (width 0.2) (layer "F.Cu") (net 5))
 (segment (start 116.588 81.4683) (end 116.3 81.4683) (width 0.2) (layer "F.Cu") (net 5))
 (segment (start 111.4 72.46) (end 115.1483 72.46) (width 0.2) (layer "B.Cu") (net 6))
 (segment (start 111.4 76.76) (end 111.4 72.46) (width 0.2) (layer "B.Cu") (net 6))
 (segment (start 116.3 72.46) (end 115.1483 72.46) (width 0.2) (layer "B.Cu") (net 6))
 (segment (start 111.4 72.46) (end 111.4 72.4) (width 0.2) (layer "B.Cu") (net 6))
 (segment (start 116.3 77.54) (end 117.4517 77.54) (width 0.2) (layer "B.Cu") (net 2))
 (segment (start 121.5917 81.68) (end 117.4517 77.54) (width 0.2) (layer "B.Cu") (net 2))
 (segment (start 123.56 81.68) (end 121.5917 81.68) (width 0.2) (layer "B.Cu") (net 2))
 (segment (start 111.4 81.84) (end 113.16 80.08) (width 0.2) (layer "F.Cu") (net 7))
 (segment (start 113.16 80.08) (end 116.3 80.08) (width 0.2) (layer "F.Cu") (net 7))
 (segment (start 121.5917 84.22) (end 117.4517 80.08) (width 0.2) (layer "B.Cu") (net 7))
 (segment (start 116.3 80.08) (end 117.4517 80.08) (width 0.2) (layer "B.Cu") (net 7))
 (segment (start 123.56 84.22) (end 121.5917 84.22) (width 0.2) (layer "B.Cu") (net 7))
 (segment (start 117.6898 74.9057) (end 117.6898 72.193) (width 0.2) (layer "B.Cu") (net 4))
 (segment (start 124.83 82.95) (end 124.83 81.2616) (width 0.2) (layer "B.Cu") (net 4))
 (segment (start 123.9784 80.41) (end 123.1941 80.41) (width 0.2) (layer "B.Cu") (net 4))
 (segment (start 124.83 81.2616) (end 123.9784 80.41) (width 0.2) (layer "B.Cu") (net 4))
 (segment (start 116.3 69.92) (end 116.3 71.0717) (width 0.2) (layer "B.Cu") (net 4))
 (segment (start 123.1941 80.41) (end 117.6898 74.9057) (width 0.2) (layer "B.Cu") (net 4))
 (segment (start 116.5685 71.0717) (end 116.3 71.0717) (width 0.2) (layer "B.Cu") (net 4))
 (segment (start 126.1 84.22) (end 124.83 82.95) (width 0.2) (layer "B.Cu") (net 4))
 (segment (start 117.6898 72.193) (end 116.5685 71.0717) (width 0.2) (layer "B.Cu") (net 4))
 (segment (start 133.36 63.35) (end 133.36 58.7) (width 0.2) (layer "F.Cu") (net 1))
 (segment (start 117.8699 67.7982) (end 132.0065 67.7982) (width 0.2) (layer "F.Cu") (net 1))
 (segment (start 133.36 68) (end 132.2083 68) (width 0.2) (layer "F.Cu") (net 1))
 (segment (start 117.4517 67.38) (end 117.8699 67.7982) (width 0.2) (layer "F.Cu") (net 1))
 (segment (start 132.0065 67.7982) (end 132.2083 68) (width 0.2) (layer "F.Cu") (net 1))
 (segment (start 116.3 67.38) (end 117.4517 67.38) (width 0.2) (layer "F.Cu") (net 1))
 (segment (start 133.36 82.5258) (end 133.36 81.95) (width 0.2) (layer "B.Cu") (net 1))
 (segment (start 133.36 72.65) (end 133.36 68) (width 0.2) (layer "B.Cu") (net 1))
 (segment (start 133.36 86.6) (end 133.36 83.1017) (width 0.2) (layer "B.Cu") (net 1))
 (segment (start 133.36 68) (end 133.36 63.35) (width 0.2) (layer "B.Cu") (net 1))
 (segment (start 133.36 77.3) (end 133.36 72.65) (width 0.2) (layer "B.Cu") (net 1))
 (segment (start 133.36 91.25) (end 133.36 86.6) (width 0.2) (layer "B.Cu") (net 1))
 (segment (start 133.36 82.5258) (end 133.36 83.1017) (width 0.2) (layer "B.Cu") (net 1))
 (segment (start 133.36 81.95) (end 133.36 77.3) (width 0.2) (layer "B.Cu") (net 1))
 (segment (start 131.3253 75.1165) (end 126.5771 70.3683) (width 0.2) (layer "F.Cu") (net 14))
 (segment (start 137.0517 79.6466) (end 137.0517 76.3183) (width 0.2) (layer "F.Cu") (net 14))
 (segment (start 124.9483 70.3683) (end 123.56 68.98) (width 0.2) (layer "F.Cu") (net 14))
 (segment (start 135.8499 75.1165) (end 131.3253 75.1165) (width 0.2) (layer "F.Cu") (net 14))
 (segment (start 135.9 80.7983) (end 137.0517 79.6466) (width 0.2) (layer "F.Cu") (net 14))
 (segment (start 126.5771 70.3683) (end 124.9483 70.3683) (width 0.2) (layer "F.Cu") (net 14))
 (segment (start 137.0517 76.3183) (end 135.8499 75.1165) (width 0.2) (layer "F.Cu") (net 14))
 (segment (start 135.9 81.95) (end 135.9 80.7983) (width 0.2) (layer "F.Cu") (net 14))
 (segment (start 134.7483 77.5879) (end 133.8779 78.4583) (width 0.2) (layer "F.Cu") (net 10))
 (segment (start 133.8779 78.4583) (end 132.6783 78.4583) (width 0.2) (layer "F.Cu") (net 10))
 (segment (start 124.7565 77.9435) (end 123.56 79.14) (width 0.2) (layer "F.Cu") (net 10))
 (segment (start 132.6783 78.4583) (end 132.1635 77.9435) (width 0.2) (layer "F.Cu") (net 10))
 (segment (start 132.1635 77.9435) (end 124.7565 77.9435) (width 0.2) (layer "F.Cu") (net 10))
 (segment (start 134.7483 77.3) (end 134.7483 77.5879) (width 0.2) (layer "F.Cu") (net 10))
 (segment (start 135.9 77.3) (end 134.7483 77.3) (width 0.2) (layer "F.Cu") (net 10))
 (segment (start 135.9 72.65) (end 134.7483 72.65) (width 0.2) (layer "F.Cu") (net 8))
 (segment (start 131.3662 68.98) (end 134.7483 72.3621) (width 0.2) (layer "F.Cu") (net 8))
 (segment (start 126.1 68.98) (end 131.3662 68.98) (width 0.2) (layer "F.Cu") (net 8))
 (segment (start 134.7483 72.3621) (end 134.7483 72.65) (width 0.2) (layer "F.Cu") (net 8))
 (segment (start 133.8846 64.5017) (end 134.7483 63.638) (width 0.2) (layer "F.Cu") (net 12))
 (segment (start 125.4983 64.5017) (end 133.8846 64.5017) (width 0.2) (layer "F.Cu") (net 12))
 (segment (start 135.9 63.35) (end 134.7483 63.35) (width 0.2) (layer "F.Cu") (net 12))
 (segment (start 134.7483 63.638) (end 134.7483 63.35) (width 0.2) (layer "F.Cu") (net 12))
 (segment (start 123.56 66.44) (end 125.4983 64.5017) (width 0.2) (layer "F.Cu") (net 12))
 (segment (start 124.83 77.87) (end 124.83 67.71) (width 0.2) (layer "B.Cu") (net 12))
 (segment (start 126.1 79.14) (end 124.83 77.87) (width 0.2) (layer "B.Cu") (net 12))
 (segment (start 124.83 67.71) (end 123.56 66.44) (width 0.2) (layer "B.Cu") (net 12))
 (segment (start 128.5174 59.8517) (end 133.8846 59.8517) (width 0.2) (layer "B.Cu") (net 18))
 (segment (start 122.3908 75.4308) (end 122.3908 65.9783) (width 0.2) (layer "B.Cu") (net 18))
 (segment (start 134.7483 58.988) (end 134.7483 58.7) (width 0.2) (layer "B.Cu") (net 18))
 (segment (start 123.56 76.6) (end 122.3908 75.4308) (width 0.2) (layer "B.Cu") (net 18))
 (segment (start 135.9 58.7) (end 134.7483 58.7) (width 0.2) (layer "B.Cu") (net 18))
 (segment (start 122.3908 65.9783) (end 128.5174 59.8517) (width 0.2) (layer "B.Cu") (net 18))
 (segment (start 133.8846 59.8517) (end 134.7483 58.988) (width 0.2) (layer "B.Cu") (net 18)))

